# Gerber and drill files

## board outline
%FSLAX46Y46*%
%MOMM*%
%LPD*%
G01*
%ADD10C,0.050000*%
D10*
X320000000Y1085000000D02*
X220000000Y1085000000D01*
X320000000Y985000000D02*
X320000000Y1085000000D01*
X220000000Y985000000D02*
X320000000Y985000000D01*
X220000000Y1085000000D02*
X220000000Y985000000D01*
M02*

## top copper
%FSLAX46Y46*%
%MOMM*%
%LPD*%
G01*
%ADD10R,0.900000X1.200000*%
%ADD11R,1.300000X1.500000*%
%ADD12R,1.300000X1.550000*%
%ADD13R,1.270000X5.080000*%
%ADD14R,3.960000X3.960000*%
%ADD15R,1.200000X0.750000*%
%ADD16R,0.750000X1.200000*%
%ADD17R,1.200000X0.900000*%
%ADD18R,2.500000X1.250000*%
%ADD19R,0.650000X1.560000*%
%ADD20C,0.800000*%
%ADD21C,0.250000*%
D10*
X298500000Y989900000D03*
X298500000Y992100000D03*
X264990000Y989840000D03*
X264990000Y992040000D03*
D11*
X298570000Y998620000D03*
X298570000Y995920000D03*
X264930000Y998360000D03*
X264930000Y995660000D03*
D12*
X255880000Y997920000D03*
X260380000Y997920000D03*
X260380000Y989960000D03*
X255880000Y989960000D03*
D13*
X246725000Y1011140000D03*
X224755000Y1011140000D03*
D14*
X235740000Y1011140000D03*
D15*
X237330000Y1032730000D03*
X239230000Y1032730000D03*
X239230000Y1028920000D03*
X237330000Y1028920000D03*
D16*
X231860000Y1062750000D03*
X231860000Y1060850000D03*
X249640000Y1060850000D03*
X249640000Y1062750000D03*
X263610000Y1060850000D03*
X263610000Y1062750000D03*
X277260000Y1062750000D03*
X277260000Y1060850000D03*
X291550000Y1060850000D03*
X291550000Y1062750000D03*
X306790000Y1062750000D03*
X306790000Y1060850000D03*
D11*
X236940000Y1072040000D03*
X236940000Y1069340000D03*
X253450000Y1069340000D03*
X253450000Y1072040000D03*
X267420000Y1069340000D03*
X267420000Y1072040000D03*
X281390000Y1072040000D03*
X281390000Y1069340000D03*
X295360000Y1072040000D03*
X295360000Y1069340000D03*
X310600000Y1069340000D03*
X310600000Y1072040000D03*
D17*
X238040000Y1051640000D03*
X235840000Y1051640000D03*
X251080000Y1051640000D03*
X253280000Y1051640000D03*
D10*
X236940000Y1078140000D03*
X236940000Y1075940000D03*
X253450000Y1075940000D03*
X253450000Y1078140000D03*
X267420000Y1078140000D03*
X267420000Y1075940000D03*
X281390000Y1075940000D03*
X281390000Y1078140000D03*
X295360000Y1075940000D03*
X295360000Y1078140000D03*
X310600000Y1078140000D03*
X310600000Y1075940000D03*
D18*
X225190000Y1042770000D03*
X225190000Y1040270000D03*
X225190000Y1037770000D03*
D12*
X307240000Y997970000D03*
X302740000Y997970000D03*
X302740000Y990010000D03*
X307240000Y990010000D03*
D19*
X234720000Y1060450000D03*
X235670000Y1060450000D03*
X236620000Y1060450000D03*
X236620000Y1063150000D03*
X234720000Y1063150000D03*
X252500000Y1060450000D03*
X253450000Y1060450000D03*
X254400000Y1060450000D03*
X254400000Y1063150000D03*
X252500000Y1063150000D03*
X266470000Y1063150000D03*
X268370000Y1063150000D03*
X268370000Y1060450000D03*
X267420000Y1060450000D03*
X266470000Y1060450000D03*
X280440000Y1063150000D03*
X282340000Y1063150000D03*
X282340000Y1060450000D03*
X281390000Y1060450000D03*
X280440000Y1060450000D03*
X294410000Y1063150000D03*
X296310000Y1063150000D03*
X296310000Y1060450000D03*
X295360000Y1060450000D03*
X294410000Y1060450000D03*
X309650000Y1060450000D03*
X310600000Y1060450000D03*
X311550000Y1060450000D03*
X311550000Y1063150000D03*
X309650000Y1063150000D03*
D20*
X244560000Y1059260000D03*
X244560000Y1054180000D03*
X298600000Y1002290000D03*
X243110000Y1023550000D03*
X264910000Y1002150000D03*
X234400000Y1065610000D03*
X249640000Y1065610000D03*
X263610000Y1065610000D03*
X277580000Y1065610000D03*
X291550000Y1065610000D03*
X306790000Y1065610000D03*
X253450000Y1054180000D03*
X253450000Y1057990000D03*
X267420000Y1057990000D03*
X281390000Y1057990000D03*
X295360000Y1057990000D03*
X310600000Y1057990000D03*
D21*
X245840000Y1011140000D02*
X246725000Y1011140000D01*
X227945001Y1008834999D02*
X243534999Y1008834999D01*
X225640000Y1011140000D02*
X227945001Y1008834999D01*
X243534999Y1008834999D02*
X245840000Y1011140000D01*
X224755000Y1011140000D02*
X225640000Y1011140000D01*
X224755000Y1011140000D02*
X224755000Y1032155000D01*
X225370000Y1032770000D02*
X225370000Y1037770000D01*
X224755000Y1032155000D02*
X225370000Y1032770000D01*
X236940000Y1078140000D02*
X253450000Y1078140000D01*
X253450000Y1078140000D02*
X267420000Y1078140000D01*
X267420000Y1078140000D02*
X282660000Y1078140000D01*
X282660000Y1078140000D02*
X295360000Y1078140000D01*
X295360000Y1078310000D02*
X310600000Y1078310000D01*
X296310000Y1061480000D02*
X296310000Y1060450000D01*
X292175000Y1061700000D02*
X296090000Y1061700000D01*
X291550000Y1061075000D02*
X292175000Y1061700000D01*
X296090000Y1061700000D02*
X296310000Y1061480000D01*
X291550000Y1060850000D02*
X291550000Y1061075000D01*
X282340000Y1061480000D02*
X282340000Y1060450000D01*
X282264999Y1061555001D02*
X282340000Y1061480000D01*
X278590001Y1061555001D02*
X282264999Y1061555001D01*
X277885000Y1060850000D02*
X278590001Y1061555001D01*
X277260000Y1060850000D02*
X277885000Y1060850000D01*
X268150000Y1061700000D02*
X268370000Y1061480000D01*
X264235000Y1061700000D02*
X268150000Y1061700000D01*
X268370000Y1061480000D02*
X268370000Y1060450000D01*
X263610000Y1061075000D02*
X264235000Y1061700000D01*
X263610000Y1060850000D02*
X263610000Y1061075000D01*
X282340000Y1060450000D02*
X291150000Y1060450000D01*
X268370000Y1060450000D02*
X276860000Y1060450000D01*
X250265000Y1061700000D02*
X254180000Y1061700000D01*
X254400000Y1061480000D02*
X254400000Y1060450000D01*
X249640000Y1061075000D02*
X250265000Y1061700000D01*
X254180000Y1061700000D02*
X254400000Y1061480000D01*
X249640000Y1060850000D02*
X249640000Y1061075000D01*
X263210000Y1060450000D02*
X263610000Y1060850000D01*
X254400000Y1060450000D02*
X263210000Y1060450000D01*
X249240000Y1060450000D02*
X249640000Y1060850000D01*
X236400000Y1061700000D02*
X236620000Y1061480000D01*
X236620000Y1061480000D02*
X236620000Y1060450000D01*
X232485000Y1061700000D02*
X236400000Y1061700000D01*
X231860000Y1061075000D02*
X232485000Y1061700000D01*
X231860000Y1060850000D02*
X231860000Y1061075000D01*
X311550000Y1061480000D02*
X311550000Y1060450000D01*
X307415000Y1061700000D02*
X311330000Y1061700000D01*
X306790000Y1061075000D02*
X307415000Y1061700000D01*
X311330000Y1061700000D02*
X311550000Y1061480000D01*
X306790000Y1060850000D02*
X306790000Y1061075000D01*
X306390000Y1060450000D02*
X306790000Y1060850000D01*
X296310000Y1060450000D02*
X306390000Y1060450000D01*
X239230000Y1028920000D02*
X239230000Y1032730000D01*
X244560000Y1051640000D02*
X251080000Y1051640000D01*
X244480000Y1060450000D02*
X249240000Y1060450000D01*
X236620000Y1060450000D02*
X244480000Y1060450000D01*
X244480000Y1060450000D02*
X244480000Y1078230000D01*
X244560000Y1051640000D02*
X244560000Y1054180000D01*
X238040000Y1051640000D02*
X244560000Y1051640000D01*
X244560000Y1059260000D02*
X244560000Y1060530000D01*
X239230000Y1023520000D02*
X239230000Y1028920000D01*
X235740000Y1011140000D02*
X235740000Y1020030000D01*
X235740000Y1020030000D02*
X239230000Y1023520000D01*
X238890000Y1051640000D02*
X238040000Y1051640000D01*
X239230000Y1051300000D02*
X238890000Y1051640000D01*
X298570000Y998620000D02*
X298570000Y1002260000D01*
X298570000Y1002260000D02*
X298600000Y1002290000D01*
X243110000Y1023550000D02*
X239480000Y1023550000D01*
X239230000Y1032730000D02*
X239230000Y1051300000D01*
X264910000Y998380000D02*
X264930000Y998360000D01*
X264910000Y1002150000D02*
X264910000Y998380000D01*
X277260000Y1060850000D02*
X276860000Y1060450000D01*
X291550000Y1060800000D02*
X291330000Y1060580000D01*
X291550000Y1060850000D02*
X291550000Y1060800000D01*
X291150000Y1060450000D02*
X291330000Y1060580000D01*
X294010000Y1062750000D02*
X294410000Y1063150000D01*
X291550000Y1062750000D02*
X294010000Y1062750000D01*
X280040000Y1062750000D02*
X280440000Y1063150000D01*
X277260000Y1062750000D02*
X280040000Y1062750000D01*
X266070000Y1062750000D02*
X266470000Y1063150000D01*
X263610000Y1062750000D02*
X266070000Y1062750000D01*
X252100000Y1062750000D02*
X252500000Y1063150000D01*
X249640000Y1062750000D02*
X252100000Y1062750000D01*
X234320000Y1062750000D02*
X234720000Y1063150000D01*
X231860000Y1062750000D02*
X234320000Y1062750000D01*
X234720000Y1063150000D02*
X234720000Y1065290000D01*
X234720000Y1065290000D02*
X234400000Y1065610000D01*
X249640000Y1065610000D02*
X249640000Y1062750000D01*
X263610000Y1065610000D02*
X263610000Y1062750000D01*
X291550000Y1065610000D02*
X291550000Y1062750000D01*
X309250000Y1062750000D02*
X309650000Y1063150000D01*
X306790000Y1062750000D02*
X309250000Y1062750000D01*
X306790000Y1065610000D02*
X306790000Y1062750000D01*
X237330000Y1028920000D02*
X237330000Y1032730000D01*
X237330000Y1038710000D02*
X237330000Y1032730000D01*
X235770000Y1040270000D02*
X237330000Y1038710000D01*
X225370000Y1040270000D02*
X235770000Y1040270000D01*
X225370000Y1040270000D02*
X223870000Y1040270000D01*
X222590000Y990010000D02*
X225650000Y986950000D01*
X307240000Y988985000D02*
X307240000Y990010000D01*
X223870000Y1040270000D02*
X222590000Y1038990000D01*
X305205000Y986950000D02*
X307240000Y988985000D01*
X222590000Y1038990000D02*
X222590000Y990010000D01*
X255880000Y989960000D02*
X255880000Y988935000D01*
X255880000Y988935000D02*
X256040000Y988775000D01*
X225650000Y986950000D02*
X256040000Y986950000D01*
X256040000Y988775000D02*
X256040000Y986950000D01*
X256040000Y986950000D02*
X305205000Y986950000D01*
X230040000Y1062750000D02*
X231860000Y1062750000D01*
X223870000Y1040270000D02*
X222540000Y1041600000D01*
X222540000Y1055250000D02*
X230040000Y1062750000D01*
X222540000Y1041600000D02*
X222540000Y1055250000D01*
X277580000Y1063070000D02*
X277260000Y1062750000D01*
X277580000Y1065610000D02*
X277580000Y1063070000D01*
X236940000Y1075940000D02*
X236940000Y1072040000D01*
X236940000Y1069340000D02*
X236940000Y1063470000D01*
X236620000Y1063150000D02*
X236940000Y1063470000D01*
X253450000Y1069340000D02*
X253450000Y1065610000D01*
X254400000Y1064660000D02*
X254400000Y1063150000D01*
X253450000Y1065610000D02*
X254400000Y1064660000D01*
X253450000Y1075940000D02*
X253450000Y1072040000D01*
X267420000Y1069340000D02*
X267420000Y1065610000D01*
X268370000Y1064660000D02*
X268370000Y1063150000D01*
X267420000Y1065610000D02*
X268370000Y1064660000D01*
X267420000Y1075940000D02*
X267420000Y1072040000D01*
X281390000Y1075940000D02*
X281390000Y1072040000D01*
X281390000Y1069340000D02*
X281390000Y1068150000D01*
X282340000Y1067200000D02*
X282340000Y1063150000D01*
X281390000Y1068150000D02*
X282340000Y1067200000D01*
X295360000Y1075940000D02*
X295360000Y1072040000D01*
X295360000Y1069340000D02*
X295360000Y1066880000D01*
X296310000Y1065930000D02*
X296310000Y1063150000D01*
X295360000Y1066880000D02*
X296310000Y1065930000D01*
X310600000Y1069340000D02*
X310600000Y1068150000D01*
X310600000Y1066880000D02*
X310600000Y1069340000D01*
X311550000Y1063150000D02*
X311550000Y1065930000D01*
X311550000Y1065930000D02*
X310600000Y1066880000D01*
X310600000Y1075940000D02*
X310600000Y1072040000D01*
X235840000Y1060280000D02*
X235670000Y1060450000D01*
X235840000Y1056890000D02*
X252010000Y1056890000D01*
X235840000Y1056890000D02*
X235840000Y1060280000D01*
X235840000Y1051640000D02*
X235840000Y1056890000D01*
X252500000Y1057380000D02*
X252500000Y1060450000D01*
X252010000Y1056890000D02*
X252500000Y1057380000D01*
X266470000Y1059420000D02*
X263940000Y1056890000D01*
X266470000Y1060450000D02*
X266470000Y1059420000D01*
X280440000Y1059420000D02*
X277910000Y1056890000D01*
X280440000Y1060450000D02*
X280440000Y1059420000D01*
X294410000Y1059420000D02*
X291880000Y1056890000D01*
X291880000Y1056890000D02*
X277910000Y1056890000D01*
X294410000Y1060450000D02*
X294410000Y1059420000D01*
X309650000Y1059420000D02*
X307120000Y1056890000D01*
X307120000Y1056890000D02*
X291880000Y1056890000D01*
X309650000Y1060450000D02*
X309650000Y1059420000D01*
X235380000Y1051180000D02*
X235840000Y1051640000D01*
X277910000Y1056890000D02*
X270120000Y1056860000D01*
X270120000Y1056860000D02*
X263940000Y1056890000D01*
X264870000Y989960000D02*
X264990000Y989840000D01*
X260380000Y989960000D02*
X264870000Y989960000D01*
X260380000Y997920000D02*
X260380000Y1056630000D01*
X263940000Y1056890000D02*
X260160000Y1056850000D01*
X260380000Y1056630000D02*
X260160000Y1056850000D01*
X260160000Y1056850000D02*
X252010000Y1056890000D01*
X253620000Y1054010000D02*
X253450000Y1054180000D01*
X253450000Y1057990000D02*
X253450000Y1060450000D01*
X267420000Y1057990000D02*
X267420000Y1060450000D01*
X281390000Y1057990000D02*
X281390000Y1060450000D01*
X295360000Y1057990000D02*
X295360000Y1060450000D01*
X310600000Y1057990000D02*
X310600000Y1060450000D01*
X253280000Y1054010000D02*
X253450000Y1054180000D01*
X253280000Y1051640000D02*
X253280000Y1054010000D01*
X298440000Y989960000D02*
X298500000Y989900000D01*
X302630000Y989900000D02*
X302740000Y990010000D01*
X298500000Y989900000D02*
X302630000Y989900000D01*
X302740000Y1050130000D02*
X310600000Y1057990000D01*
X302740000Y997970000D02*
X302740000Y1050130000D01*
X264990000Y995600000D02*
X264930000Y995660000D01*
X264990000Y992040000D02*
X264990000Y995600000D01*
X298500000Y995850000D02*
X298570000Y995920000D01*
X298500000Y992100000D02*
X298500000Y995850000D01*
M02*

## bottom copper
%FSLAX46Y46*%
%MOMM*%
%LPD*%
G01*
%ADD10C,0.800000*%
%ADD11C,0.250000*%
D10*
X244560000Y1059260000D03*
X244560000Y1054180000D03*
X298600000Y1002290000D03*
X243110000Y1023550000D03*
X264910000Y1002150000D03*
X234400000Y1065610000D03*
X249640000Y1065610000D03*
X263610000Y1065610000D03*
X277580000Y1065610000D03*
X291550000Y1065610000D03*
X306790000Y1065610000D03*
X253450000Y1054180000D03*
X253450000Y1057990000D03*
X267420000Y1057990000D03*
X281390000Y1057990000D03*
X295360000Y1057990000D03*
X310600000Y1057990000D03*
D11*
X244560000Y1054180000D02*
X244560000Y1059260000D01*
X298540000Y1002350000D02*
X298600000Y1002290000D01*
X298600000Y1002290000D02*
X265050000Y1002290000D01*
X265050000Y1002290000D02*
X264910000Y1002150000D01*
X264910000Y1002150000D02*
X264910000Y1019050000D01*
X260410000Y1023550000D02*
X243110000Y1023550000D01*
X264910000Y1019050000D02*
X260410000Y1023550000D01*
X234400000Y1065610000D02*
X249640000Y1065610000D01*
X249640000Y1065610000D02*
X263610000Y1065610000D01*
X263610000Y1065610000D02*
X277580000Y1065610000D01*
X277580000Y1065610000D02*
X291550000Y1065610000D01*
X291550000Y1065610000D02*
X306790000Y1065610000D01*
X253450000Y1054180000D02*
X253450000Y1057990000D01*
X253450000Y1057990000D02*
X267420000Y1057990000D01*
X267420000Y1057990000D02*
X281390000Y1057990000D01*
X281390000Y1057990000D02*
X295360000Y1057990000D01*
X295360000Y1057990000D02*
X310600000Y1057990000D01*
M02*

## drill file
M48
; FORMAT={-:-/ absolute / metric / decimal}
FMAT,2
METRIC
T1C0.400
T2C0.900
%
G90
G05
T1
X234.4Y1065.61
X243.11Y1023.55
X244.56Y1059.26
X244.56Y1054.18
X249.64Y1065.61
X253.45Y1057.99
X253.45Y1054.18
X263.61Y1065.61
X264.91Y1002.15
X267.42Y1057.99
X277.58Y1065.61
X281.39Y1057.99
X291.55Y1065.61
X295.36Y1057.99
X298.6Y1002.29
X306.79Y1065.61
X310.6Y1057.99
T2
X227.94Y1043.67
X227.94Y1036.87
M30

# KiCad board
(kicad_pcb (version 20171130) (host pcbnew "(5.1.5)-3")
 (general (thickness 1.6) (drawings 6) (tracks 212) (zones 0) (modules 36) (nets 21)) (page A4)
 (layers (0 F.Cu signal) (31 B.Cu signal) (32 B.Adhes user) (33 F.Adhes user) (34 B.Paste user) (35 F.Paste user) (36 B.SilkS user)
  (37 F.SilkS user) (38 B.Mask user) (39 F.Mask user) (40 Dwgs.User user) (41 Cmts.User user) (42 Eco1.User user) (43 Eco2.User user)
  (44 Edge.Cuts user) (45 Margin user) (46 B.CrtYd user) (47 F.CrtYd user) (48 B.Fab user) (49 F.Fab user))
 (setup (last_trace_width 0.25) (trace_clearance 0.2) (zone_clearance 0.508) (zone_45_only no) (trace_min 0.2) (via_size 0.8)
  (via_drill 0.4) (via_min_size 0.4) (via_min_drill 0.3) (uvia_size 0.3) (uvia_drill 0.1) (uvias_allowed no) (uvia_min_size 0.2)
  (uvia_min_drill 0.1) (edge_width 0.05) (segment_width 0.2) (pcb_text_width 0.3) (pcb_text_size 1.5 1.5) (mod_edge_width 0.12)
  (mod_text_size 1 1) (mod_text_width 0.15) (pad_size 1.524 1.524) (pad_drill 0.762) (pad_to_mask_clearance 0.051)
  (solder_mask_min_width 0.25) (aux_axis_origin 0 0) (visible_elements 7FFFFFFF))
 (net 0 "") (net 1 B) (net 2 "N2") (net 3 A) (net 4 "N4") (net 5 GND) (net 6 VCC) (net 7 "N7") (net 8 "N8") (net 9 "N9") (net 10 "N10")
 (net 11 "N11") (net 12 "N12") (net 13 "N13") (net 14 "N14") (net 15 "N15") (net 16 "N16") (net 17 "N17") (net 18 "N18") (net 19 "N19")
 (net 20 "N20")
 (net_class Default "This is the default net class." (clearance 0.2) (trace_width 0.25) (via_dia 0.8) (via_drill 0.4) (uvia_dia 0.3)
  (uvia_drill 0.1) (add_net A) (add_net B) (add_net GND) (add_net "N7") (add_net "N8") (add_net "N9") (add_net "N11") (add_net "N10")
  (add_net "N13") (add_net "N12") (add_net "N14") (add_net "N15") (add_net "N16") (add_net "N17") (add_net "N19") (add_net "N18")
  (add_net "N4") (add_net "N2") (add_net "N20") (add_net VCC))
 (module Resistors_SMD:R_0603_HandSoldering (layer F.Cu) (at 298.5 -991 90)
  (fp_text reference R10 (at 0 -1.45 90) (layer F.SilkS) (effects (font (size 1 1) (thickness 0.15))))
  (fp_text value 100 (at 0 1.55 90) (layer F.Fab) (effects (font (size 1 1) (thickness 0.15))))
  (pad 1 smd rect (at -1.1 0 90) (size 1.2 0.9) (layers F.Cu F.Paste F.Mask) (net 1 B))
  (pad 2 smd rect (at 1.1 0 90) (size 1.2 0.9) (layers F.Cu F.Paste F.Mask) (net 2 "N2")))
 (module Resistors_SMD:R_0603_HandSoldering (layer F.Cu) (at 264.99 -990.94 90)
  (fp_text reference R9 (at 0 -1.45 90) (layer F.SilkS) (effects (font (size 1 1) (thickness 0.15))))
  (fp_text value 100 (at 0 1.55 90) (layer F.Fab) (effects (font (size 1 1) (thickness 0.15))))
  (pad 1 smd rect (at -1.1 0 90) (size 1.2 0.9) (layers F.Cu F.Paste F.Mask) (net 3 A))
  (pad 2 smd rect (at 1.1 0 90) (size 1.2 0.9) (layers F.Cu F.Paste F.Mask) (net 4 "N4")))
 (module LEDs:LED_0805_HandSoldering (layer F.Cu) (at 298.57 -997.27 270)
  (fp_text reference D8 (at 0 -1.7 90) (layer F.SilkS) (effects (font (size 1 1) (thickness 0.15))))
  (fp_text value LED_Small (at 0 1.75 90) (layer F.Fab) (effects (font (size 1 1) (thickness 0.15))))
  (pad 1 smd rect (at -1.35 0 270) (size 1.5 1.3) (layers F.Cu F.Paste F.Mask) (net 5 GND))
  (pad 2 smd rect (at 1.35 0 270) (size 1.5 1.3) (layers F.Cu F.Paste F.Mask) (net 2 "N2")))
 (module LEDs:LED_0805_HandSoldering (layer F.Cu) (at 264.93 -997.01 270)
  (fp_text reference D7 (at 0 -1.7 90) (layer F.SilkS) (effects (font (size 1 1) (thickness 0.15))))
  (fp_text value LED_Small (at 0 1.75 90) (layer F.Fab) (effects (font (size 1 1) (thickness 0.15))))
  (pad 1 smd rect (at -1.35 0 270) (size 1.5 1.3) (layers F.Cu F.Paste F.Mask) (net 5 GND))
  (pad 2 smd rect (at 1.35 0 270) (size 1.5 1.3) (layers F.Cu F.Paste F.Mask) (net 4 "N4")))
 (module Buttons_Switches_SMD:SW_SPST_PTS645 (layer F.Cu) (at 258.13 -993.94 270)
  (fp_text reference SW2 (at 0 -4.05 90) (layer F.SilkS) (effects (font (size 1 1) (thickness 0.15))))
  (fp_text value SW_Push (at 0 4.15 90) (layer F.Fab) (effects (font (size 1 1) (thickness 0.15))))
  (pad 2 smd rect (at -3.98 2.25 270) (size 1.55 1.3) (layers F.Cu F.Paste F.Mask) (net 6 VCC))
  (pad 1 smd rect (at -3.98 -2.25 270) (size 1.55 1.3) (layers F.Cu F.Paste F.Mask) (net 3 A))
  (pad 1 smd rect (at 3.98 -2.25 270) (size 1.55 1.3) (layers F.Cu F.Paste F.Mask) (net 3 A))
  (pad 2 smd rect (at 3.98 2.25 270) (size 1.55 1.3) (layers F.Cu F.Paste F.Mask) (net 6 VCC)))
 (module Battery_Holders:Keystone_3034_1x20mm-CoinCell (layer F.Cu) (at 235.74 -1011.14 180)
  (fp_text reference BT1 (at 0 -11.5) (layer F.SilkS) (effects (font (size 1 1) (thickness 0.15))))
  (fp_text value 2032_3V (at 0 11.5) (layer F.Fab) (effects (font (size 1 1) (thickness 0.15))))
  (pad 1 smd rect (at -10.985 0 180) (size 1.27 5.08) (layers F.Cu F.Paste F.Mask) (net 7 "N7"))
  (pad 1 smd rect (at 10.985 0 180) (size 1.27 5.08) (layers F.Cu F.Paste F.Mask) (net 7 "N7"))
  (pad 2 smd rect (at 0 0 180) (size 3.96 3.96) (layers F.Cu F.Paste F.Mask) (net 5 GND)))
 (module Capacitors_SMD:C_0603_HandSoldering (layer F.Cu) (at 238.28 -1032.73)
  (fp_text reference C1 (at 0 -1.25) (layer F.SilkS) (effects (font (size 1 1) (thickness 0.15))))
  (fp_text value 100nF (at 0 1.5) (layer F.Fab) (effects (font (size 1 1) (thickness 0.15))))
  (pad 1 smd rect (at -0.95 0) (size 1.2 0.75) (layers F.Cu F.Paste F.Mask) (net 6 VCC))
  (pad 2 smd rect (at 0.95 0) (size 1.2 0.75) (layers F.Cu F.Paste F.Mask) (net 5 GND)))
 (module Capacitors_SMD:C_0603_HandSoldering (layer F.Cu) (at 238.28 -1028.92)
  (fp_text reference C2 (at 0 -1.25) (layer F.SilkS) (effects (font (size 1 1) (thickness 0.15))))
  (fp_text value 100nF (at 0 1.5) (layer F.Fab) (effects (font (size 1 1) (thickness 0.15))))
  (pad 2 smd rect (at 0.95 0) (size 1.2 0.75) (layers F.Cu F.Paste F.Mask) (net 5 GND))
  (pad 1 smd rect (at -0.95 0) (size 1.2 0.75) (layers F.Cu F.Paste F.Mask) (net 6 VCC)))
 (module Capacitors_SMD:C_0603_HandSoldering (layer F.Cu) (at 231.86 -1061.8 270)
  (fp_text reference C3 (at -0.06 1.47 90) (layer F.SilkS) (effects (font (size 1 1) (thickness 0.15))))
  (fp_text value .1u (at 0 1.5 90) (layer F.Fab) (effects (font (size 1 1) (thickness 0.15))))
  (pad 1 smd rect (at -0.95 0 270) (size 1.2 0.75) (layers F.Cu F.Paste F.Mask) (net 6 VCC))
  (pad 2 smd rect (at 0.95 0 270) (size 1.2 0.75) (layers F.Cu F.Paste F.Mask) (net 5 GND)))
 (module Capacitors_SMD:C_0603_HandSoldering (layer F.Cu) (at 249.64 -1061.8 270)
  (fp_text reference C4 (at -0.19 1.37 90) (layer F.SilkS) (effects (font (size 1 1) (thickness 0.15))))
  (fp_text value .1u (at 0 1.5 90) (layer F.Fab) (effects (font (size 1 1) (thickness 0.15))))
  (pad 2 smd rect (at 0.95 0 270) (size 1.2 0.75) (layers F.Cu F.Paste F.Mask) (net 5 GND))
  (pad 1 smd rect (at -0.95 0 270) (size 1.2 0.75) (layers F.Cu F.Paste F.Mask) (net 6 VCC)))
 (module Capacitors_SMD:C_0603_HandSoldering (layer F.Cu) (at 263.61 -1061.8 270)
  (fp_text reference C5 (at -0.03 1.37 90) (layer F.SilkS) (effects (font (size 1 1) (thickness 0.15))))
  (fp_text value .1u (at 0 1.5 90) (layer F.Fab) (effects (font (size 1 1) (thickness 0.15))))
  (pad 2 smd rect (at 0.95 0 270) (size 1.2 0.75) (layers F.Cu F.Paste F.Mask) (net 5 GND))
  (pad 1 smd rect (at -0.95 0 270) (size 1.2 0.75) (layers F.Cu F.Paste F.Mask) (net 6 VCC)))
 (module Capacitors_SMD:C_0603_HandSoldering (layer F.Cu) (at 277.26 -1061.8 270)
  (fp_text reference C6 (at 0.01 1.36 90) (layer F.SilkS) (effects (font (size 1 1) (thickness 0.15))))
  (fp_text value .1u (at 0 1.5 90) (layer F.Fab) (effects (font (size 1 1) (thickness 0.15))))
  (pad 1 smd rect (at -0.95 0 270) (size 1.2 0.75) (layers F.Cu F.Paste F.Mask) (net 6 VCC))
  (pad 2 smd rect (at 0.95 0 270) (size 1.2 0.75) (layers F.Cu F.Paste F.Mask) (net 5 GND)))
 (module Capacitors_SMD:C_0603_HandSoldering (layer F.Cu) (at 291.55 -1061.8 270)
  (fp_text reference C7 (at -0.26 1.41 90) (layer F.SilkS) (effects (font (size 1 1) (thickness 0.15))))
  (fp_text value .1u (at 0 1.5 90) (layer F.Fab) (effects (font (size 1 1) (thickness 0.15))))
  (pad 2 smd rect (at 0.95 0 270) (size 1.2 0.75) (layers F.Cu F.Paste F.Mask) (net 5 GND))
  (pad 1 smd rect (at -0.95 0 270) (size 1.2 0.75) (layers F.Cu F.Paste F.Mask) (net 6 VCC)))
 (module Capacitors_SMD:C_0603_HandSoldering (layer F.Cu) (at 306.79 -1061.8 270)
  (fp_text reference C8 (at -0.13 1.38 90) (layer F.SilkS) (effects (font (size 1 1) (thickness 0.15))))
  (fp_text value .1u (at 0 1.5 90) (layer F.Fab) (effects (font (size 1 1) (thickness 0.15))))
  (pad 1 smd rect (at -0.95 0 270) (size 1.2 0.75) (layers F.Cu F.Paste F.Mask) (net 6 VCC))
  (pad 2 smd rect (at 0.95 0 270) (size 1.2 0.75) (layers F.Cu F.Paste F.Mask) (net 5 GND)))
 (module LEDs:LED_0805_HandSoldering (layer F.Cu) (at 236.94 -1070.69 270)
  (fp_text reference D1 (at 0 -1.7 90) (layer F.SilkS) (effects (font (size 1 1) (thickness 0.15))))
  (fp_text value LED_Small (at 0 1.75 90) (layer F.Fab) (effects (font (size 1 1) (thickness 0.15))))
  (pad 1 smd rect (at -1.35 0 270) (size 1.5 1.3) (layers F.Cu F.Paste F.Mask) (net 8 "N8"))
  (pad 2 smd rect (at 1.35 0 270) (size 1.5 1.3) (layers F.Cu F.Paste F.Mask) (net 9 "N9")))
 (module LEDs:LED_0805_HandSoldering (layer F.Cu) (at 253.45 -1070.69 270)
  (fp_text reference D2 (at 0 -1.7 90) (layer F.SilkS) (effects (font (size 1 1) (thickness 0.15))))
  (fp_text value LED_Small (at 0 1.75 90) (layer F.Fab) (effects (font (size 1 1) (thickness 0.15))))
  (pad 2 smd rect (at 1.35 0 270) (size 1.5 1.3) (layers F.Cu F.Paste F.Mask) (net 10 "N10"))
  (pad 1 smd rect (at -1.35 0 270) (size 1.5 1.3) (layers F.Cu F.Paste F.Mask) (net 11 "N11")))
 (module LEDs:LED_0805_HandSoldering (layer F.Cu) (at 267.42 -1070.69 270)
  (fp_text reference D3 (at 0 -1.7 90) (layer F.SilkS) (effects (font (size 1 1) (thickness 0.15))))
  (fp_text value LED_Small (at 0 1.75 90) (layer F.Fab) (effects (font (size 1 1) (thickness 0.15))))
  (pad 2 smd rect (at 1.35 0 270) (size 1.5 1.3) (layers F.Cu F.Paste F.Mask) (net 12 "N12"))
  (pad 1 smd rect (at -1.35 0 270) (size 1.5 1.3) (layers F.Cu F.Paste F.Mask) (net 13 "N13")))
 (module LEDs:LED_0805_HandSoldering (layer F.Cu) (at 281.39 -1070.69 270)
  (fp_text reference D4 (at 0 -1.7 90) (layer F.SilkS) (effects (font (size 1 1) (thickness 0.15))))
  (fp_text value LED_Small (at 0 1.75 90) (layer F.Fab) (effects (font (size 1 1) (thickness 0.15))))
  (pad 1 smd rect (at -1.35 0 270) (size 1.5 1.3) (layers F.Cu F.Paste F.Mask) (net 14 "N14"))
  (pad 2 smd rect (at 1.35 0 270) (size 1.5 1.3) (layers F.Cu F.Paste F.Mask) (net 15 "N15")))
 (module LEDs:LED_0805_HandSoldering (layer F.Cu) (at 295.36 -1070.69 270)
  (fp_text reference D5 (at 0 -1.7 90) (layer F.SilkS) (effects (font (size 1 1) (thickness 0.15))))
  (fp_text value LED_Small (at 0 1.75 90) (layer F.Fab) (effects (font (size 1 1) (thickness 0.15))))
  (pad 1 smd rect (at -1.35 0 270) (size 1.5 1.3) (layers F.Cu F.Paste F.Mask) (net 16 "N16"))
  (pad 2 smd rect (at 1.35 0 270) (size 1.5 1.3) (layers F.Cu F.Paste F.Mask) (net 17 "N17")))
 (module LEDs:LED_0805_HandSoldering (layer F.Cu) (at 310.6 -1070.69 270)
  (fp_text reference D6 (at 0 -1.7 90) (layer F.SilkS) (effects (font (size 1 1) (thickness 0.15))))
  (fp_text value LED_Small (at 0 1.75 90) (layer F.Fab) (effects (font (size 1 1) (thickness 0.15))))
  (pad 2 smd rect (at 1.35 0 270) (size 1.5 1.3) (layers F.Cu F.Paste F.Mask) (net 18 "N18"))
  (pad 1 smd rect (at -1.35 0 270) (size 1.5 1.3) (layers F.Cu F.Paste F.Mask) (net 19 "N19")))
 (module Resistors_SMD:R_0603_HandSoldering (layer F.Cu) (at 236.94 -1051.64 180)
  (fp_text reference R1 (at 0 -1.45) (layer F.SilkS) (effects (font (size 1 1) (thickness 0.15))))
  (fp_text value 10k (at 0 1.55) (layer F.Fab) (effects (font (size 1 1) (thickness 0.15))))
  (pad 1 smd rect (at -1.1 0 180) (size 1.2 0.9) (layers F.Cu F.Paste F.Mask) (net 5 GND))
  (pad 2 smd rect (at 1.1 0 180) (size 1.2 0.9) (layers F.Cu F.Paste F.Mask) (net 3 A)))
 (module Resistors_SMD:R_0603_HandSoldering (layer F.Cu) (at 252.18 -1051.64 180)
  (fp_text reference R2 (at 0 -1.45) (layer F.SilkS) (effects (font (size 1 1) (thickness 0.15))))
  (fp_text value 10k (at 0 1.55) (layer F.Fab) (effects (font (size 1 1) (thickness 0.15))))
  (pad 2 smd rect (at 1.1 0 180) (size 1.2 0.9) (layers F.Cu F.Paste F.Mask) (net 5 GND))
  (pad 1 smd rect (at -1.1 0 180) (size 1.2 0.9) (layers F.Cu F.Paste F.Mask) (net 1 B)))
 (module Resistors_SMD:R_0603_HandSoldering (layer F.Cu) (at 236.94 -1077.04 270)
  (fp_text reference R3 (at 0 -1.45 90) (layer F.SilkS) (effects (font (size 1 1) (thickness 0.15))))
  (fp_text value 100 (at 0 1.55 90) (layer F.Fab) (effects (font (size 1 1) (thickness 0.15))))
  (pad 1 smd rect (at -1.1 0 270) (size 1.2 0.9) (layers F.Cu F.Paste F.Mask) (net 5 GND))
  (pad 2 smd rect (at 1.1 0 270) (size 1.2 0.9) (layers F.Cu F.Paste F.Mask) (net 8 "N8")))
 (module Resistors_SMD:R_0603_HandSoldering (layer F.Cu) (at 253.45 -1077.04 270)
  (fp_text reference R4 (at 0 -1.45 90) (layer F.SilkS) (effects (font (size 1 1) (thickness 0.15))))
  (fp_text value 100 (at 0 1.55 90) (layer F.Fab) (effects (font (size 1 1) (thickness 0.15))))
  (pad 2 smd rect (at 1.1 0 270) (size 1.2 0.9) (layers F.Cu F.Paste F.Mask) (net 11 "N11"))
  (pad 1 smd rect (at -1.1 0 270) (size 1.2 0.9) (layers F.Cu F.Paste F.Mask) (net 5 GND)))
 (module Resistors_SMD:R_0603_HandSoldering (layer F.Cu) (at 267.42 -1077.04 270)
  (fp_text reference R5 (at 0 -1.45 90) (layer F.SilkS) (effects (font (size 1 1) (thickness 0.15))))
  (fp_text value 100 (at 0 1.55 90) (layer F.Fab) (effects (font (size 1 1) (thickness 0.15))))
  (pad 1 smd rect (at -1.1 0 270) (size 1.2 0.9) (layers F.Cu F.Paste F.Mask) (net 5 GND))
  (pad 2 smd rect (at 1.1 0 270) (size 1.2 0.9) (layers F.Cu F.Paste F.Mask) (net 13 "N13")))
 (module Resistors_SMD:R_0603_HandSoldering (layer F.Cu) (at 281.39 -1077.04 270)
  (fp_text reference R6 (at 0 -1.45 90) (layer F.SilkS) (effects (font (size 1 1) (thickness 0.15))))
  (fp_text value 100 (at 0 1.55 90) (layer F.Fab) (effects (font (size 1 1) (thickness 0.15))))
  (pad 2 smd rect (at 1.1 0 270) (size 1.2 0.9) (layers F.Cu F.Paste F.Mask) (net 14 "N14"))
  (pad 1 smd rect (at -1.1 0 270) (size 1.2 0.9) (layers F.Cu F.Paste F.Mask) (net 5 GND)))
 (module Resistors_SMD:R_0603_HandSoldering (layer F.Cu) (at 295.36 -1077.04 270)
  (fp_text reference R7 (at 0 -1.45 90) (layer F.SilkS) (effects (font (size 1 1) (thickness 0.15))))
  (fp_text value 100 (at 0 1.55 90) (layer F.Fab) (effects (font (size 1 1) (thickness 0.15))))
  (pad 2 smd rect (at 1.1 0 270) (size 1.2 0.9) (layers F.Cu F.Paste F.Mask) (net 16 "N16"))
  (pad 1 smd rect (at -1.1 0 270) (size 1.2 0.9) (layers F.Cu F.Paste F.Mask) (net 5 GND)))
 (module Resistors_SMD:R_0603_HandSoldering (layer F.Cu) (at 310.6 -1077.04 270)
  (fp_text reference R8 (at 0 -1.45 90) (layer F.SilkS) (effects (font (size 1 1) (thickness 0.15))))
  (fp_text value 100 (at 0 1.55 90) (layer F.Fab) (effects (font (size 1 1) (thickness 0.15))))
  (pad 1 smd rect (at -1.1 0 270) (size 1.2 0.9) (layers F.Cu F.Paste F.Mask) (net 5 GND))
  (pad 2 smd rect (at 1.1 0 270) (size 1.2 0.9) (layers F.Cu F.Paste F.Mask) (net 19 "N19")))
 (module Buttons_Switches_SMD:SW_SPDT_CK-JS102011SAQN (layer F.Cu) (at 227.94 -1040.27 90)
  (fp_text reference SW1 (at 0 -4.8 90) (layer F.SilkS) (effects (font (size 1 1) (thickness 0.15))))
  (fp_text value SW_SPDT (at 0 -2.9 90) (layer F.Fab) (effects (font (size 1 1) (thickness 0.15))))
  (pad "" np_thru_hole circle (at 3.4 0 90) (size 0.9 0.9) (drill 0.9) (layers *.Cu *.Mask))
  (pad "" np_thru_hole circle (at -3.4 0 90) (size 0.9 0.9) (drill 0.9) (layers *.Cu *.Mask))
  (pad 3 smd rect (at 2.5 -2.75 90) (size 1.25 2.5) (layers F.Cu F.Paste F.Mask) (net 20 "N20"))
  (pad 2 smd rect (at 0 -2.75 90) (size 1.25 2.5) (layers F.Cu F.Paste F.Mask) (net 6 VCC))
  (pad 1 smd rect (at -2.5 -2.75 90) (size 1.25 2.5) (layers F.Cu F.Paste F.Mask) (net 7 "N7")))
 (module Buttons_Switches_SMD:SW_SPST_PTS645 (layer F.Cu) (at 304.99 -993.99 90)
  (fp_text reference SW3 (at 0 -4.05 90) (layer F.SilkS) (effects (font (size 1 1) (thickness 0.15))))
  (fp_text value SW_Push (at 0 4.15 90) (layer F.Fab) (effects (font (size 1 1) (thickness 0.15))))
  (pad 2 smd rect (at 3.98 2.25 90) (size 1.55 1.3) (layers F.Cu F.Paste F.Mask) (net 6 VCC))
  (pad 1 smd rect (at 3.98 -2.25 90) (size 1.55 1.3) (layers F.Cu F.Paste F.Mask) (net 1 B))
  (pad 1 smd rect (at -3.98 -2.25 90) (size 1.55 1.3) (layers F.Cu F.Paste F.Mask) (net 1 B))
  (pad 2 smd rect (at -3.98 2.25 90) (size 1.55 1.3) (layers F.Cu F.Paste F.Mask) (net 6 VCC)))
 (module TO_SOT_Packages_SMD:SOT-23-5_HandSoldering (layer F.Cu) (at 235.67 -1061.8 90)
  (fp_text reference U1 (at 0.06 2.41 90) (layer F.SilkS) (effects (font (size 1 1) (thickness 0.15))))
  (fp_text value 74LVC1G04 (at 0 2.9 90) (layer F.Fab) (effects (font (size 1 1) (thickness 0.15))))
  (pad 1 smd rect (at -1.35 -0.95 90) (size 1.56 0.65) (layers F.Cu F.Paste F.Mask))
  (pad 2 smd rect (at -1.35 0 90) (size 1.56 0.65) (layers F.Cu F.Paste F.Mask) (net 3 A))
  (pad 3 smd rect (at -1.35 0.95 90) (size 1.56 0.65) (layers F.Cu F.Paste F.Mask) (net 5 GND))
  (pad 4 smd rect (at 1.35 0.95 90) (size 1.56 0.65) (layers F.Cu F.Paste F.Mask) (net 9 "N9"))
  (pad 5 smd rect (at 1.35 -0.95 90) (size 1.56 0.65) (layers F.Cu F.Paste F.Mask) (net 6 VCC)))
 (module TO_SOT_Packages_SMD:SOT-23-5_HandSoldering (layer F.Cu) (at 253.45 -1061.8 90)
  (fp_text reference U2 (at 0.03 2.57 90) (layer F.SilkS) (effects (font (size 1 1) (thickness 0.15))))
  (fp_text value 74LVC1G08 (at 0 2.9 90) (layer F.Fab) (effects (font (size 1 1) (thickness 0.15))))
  (pad 1 smd rect (at -1.35 -0.95 90) (size 1.56 0.65) (layers F.Cu F.Paste F.Mask) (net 3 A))
  (pad 2 smd rect (at -1.35 0 90) (size 1.56 0.65) (layers F.Cu F.Paste F.Mask) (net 1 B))
  (pad 3 smd rect (at -1.35 0.95 90) (size 1.56 0.65) (layers F.Cu F.Paste F.Mask) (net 5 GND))
  (pad 4 smd rect (at 1.35 0.95 90) (size 1.56 0.65) (layers F.Cu F.Paste F.Mask) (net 10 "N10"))
  (pad 5 smd rect (at 1.35 -0.95 90) (size 1.56 0.65) (layers F.Cu F.Paste F.Mask) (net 6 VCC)))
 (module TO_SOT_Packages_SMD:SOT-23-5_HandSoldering (layer F.Cu) (at 267.42 -1061.8 90)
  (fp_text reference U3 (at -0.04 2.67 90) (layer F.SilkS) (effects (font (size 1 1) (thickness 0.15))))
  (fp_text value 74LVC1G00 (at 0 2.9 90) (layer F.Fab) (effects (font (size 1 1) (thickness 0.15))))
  (pad 5 smd rect (at 1.35 -0.95 90) (size 1.56 0.65) (layers F.Cu F.Paste F.Mask) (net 6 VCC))
  (pad 4 smd rect (at 1.35 0.95 90) (size 1.56 0.65) (layers F.Cu F.Paste F.Mask) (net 12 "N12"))
  (pad 3 smd rect (at -1.35 0.95 90) (size 1.56 0.65) (layers F.Cu F.Paste F.Mask) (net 5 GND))
  (pad 2 smd rect (at -1.35 0 90) (size 1.56 0.65) (layers F.Cu F.Paste F.Mask) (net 1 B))
  (pad 1 smd rect (at -1.35 -0.95 90) (size 1.56 0.65) (layers F.Cu F.Paste F.Mask) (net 3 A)))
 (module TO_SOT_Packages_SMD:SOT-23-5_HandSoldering (layer F.Cu) (at 281.39 -1061.8 90)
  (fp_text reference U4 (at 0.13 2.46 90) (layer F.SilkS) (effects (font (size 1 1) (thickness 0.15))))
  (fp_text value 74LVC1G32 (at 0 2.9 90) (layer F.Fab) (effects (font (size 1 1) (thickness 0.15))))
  (pad 5 smd rect (at 1.35 -0.95 90) (size 1.56 0.65) (layers F.Cu F.Paste F.Mask) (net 6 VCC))
  (pad 4 smd rect (at 1.35 0.95 90) (size 1.56 0.65) (layers F.Cu F.Paste F.Mask) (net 15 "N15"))
  (pad 3 smd rect (at -1.35 0.95 90) (size 1.56 0.65) (layers F.Cu F.Paste F.Mask) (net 5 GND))
  (pad 2 smd rect (at -1.35 0 90) (size 1.56 0.65) (layers F.Cu F.Paste F.Mask) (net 1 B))
  (pad 1 smd rect (at -1.35 -0.95 90) (size 1.56 0.65) (layers F.Cu F.Paste F.Mask) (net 3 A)))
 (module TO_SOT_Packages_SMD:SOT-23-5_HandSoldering (layer F.Cu) (at 295.36 -1061.8 90)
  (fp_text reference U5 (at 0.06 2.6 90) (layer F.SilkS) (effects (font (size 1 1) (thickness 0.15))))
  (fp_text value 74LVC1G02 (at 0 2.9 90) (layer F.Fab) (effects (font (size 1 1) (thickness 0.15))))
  (pad 5 smd rect (at 1.35 -0.95 90) (size 1.56 0.65) (layers F.Cu F.Paste F.Mask) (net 6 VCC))
  (pad 4 smd rect (at 1.35 0.95 90) (size 1.56 0.65) (layers F.Cu F.Paste F.Mask) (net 17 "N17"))
  (pad 3 smd rect (at -1.35 0.95 90) (size 1.56 0.65) (layers F.Cu F.Paste F.Mask) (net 5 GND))
  (pad 2 smd rect (at -1.35 0 90) (size 1.56 0.65) (layers F.Cu F.Paste F.Mask) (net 1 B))
  (pad 1 smd rect (at -1.35 -0.95 90) (size 1.56 0.65) (layers F.Cu F.Paste F.Mask) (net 3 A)))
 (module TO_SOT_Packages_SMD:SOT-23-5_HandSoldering (layer F.Cu) (at 310.6 -1061.8 90)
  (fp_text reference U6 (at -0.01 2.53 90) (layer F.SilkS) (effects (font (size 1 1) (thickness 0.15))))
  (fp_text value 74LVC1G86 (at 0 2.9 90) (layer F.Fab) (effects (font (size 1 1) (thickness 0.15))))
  (pad 1 smd rect (at -1.35 -0.95 90) (size 1.56 0.65) (layers F.Cu F.Paste F.Mask) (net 3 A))
  (pad 2 smd rect (at -1.35 0 90) (size 1.56 0.65) (layers F.Cu F.Paste F.Mask) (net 1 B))
  (pad 3 smd rect (at -1.35 0.95 90) (size 1.56 0.65) (layers F.Cu F.Paste F.Mask) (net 5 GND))
  (pad 4 smd rect (at 1.35 0.95 90) (size 1.56 0.65) (layers F.Cu F.Paste F.Mask) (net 18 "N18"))
  (pad 5 smd rect (at 1.35 -0.95 90) (size 1.56 0.65) (layers F.Cu F.Paste F.Mask) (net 6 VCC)))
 (gr_line (start 320 -1085) (end 220 -1085) (layer Edge.Cuts) (width 0.05))
 (gr_line (start 320 -985) (end 320 -1085) (layer Edge.Cuts) (width 0.05))
 (gr_line (start 220 -985) (end 320 -985) (layer Edge.Cuts) (width 0.05))
 (gr_line (start 220 -1085) (end 220 -985) (layer Edge.Cuts) (width 0.05))
 (segment (start 245.84 -1011.14) (end 246.725 -1011.14) (width 0.25) (layer F.Cu) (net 7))
 (segment (start 227.945001 -1008.834999) (end 243.534999 -1008.834999) (width 0.25) (layer F.Cu) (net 7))
 (segment (start 225.64 -1011.14) (end 227.945001 -1008.834999) (width 0.25) (layer F.Cu) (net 7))
 (segment (start 243.534999 -1008.834999) (end 245.84 -1011.14) (width 0.25) (layer F.Cu) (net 7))
 (segment (start 224.755 -1011.14) (end 225.64 -1011.14) (width 0.25) (layer F.Cu) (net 7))
 (segment (start 224.755 -1011.14) (end 224.755 -1032.155) (width 0.25) (layer F.Cu) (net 7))
 (segment (start 225.37 -1032.77) (end 225.37 -1037.77) (width 0.25) (layer F.Cu) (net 7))
 (segment (start 224.755 -1032.155) (end 225.37 -1032.77) (width 0.25) (layer F.Cu) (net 7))
 (segment (start 236.94 -1078.14) (end 253.45 -1078.14) (width 0.25) (layer F.Cu) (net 5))
 (segment (start 253.45 -1078.14) (end 267.42 -1078.14) (width 0.25) (layer F.Cu) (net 5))
 (segment (start 267.42 -1078.14) (end 282.66 -1078.14) (width 0.25) (layer F.Cu) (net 5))
 (segment (start 282.66 -1078.14) (end 295.36 -1078.14) (width 0.25) (layer F.Cu) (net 5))
 (segment (start 295.36 -1078.31) (end 310.6 -1078.31) (width 0.25) (layer F.Cu) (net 5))
 (segment (start 296.31 -1061.48) (end 296.31 -1060.45) (width 0.25) (layer F.Cu) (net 5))
 (segment (start 292.175 -1061.7) (end 296.09 -1061.7) (width 0.25) (layer F.Cu) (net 5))
 (segment (start 291.55 -1061.075) (end 292.175 -1061.7) (width 0.25) (layer F.Cu) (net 5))
 (segment (start 296.09 -1061.7) (end 296.31 -1061.48) (width 0.25) (layer F.Cu) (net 5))
 (segment (start 291.55 -1060.85) (end 291.55 -1061.075) (width 0.25) (layer F.Cu) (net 5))
 (segment (start 282.34 -1061.48) (end 282.34 -1060.45) (width 0.25) (layer F.Cu) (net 5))
 (segment (start 282.264999 -1061.555001) (end 282.34 -1061.48) (width 0.25) (layer F.Cu) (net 5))
 (segment (start 278.590001 -1061.555001) (end 282.264999 -1061.555001) (width 0.25) (layer F.Cu) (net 5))
 (segment (start 277.885 -1060.85) (end 278.590001 -1061.555001) (width 0.25) (layer F.Cu) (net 5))
 (segment (start 277.26 -1060.85) (end 277.885 -1060.85) (width 0.25) (layer F.Cu) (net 5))
 (segment (start 268.15 -1061.7) (end 268.37 -1061.48) (width 0.25) (layer F.Cu) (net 5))
 (segment (start 264.235 -1061.7) (end 268.15 -1061.7) (width 0.25) (layer F.Cu) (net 5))
 (segment (start 268.37 -1061.48) (end 268.37 -1060.45) (width 0.25) (layer F.Cu) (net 5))
 (segment (start 263.61 -1061.075) (end 264.235 -1061.7) (width 0.25) (layer F.Cu) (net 5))
 (segment (start 263.61 -1060.85) (end 263.61 -1061.075) (width 0.25) (layer F.Cu) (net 5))
 (segment (start 282.34 -1060.45) (end 291.15 -1060.45) (width 0.25) (layer F.Cu) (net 5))
 (segment (start 268.37 -1060.45) (end 276.86 -1060.45) (width 0.25) (layer F.Cu) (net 5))
 (segment (start 250.265 -1061.7) (end 254.18 -1061.7) (width 0.25) (layer F.Cu) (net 5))
 (segment (start 254.4 -1061.48) (end 254.4 -1060.45) (width 0.25) (layer F.Cu) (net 5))
 (segment (start 249.64 -1061.075) (end 250.265 -1061.7) (width 0.25) (layer F.Cu) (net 5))
 (segment (start 254.18 -1061.7) (end 254.4 -1061.48) (width 0.25) (layer F.Cu) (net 5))
 (segment (start 249.64 -1060.85) (end 249.64 -1061.075) (width 0.25) (layer F.Cu) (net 5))
 (segment (start 263.21 -1060.45) (end 263.61 -1060.85) (width 0.25) (layer F.Cu) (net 5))
 (segment (start 254.4 -1060.45) (end 263.21 -1060.45) (width 0.25) (layer F.Cu) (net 5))
 (segment (start 249.24 -1060.45) (end 249.64 -1060.85) (width 0.25) (layer F.Cu) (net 5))
 (segment (start 236.4 -1061.7) (end 236.62 -1061.48) (width 0.25) (layer F.Cu) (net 5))
 (segment (start 236.62 -1061.48) (end 236.62 -1060.45) (width 0.25) (layer F.Cu) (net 5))
 (segment (start 232.485 -1061.7) (end 236.4 -1061.7) (width 0.25) (layer F.Cu) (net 5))
 (segment (start 231.86 -1061.075) (end 232.485 -1061.7) (width 0.25) (layer F.Cu) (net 5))
 (segment (start 231.86 -1060.85) (end 231.86 -1061.075) (width 0.25) (layer F.Cu) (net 5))
 (segment (start 311.55 -1061.48) (end 311.55 -1060.45) (width 0.25) (layer F.Cu) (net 5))
 (segment (start 307.415 -1061.7) (end 311.33 -1061.7) (width 0.25) (layer F.Cu) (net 5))
 (segment (start 306.79 -1061.075) (end 307.415 -1061.7) (width 0.25) (layer F.Cu) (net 5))
 (segment (start 311.33 -1061.7) (end 311.55 -1061.48) (width 0.25) (layer F.Cu) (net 5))
 (segment (start 306.79 -1060.85) (end 306.79 -1061.075) (width 0.25) (layer F.Cu) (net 5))
 (segment (start 306.39 -1060.45) (end 306.79 -1060.85) (width 0.25) (layer F.Cu) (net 5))
 (segment (start 296.31 -1060.45) (end 306.39 -1060.45) (width 0.25) (layer F.Cu) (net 5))
 (segment (start 239.23 -1028.92) (end 239.23 -1032.73) (width 0.25) (layer F.Cu) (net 5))
 (segment (start 244.56 -1051.64) (end 251.08 -1051.64) (width 0.25) (layer F.Cu) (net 5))
 (segment (start 244.48 -1060.45) (end 249.24 -1060.45) (width 0.25) (layer F.Cu) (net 5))
 (segment (start 236.62 -1060.45) (end 244.48 -1060.45) (width 0.25) (layer F.Cu) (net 5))
 (segment (start 244.48 -1060.45) (end 244.48 -1078.23) (width 0.25) (layer F.Cu) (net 5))
 (via (at 244.56 -1059.26) (size 0.8) (drill 0.4) (layers F.Cu B.Cu) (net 5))
 (via (at 244.56 -1054.18) (size 0.8) (drill 0.4) (layers F.Cu B.Cu) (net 5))
 (segment (start 244.56 -1051.64) (end 244.56 -1054.18) (width 0.25) (layer F.Cu) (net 5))
 (segment (start 238.04 -1051.64) (end 244.56 -1051.64) (width 0.25) (layer F.Cu) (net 5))
 (segment (start 244.56 -1054.18) (end 244.56 -1059.26) (width 0.25) (layer B.Cu) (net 5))
 (segment (start 244.56 -1059.26) (end 244.56 -1060.53) (width 0.25) (layer F.Cu) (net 5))
 (segment (start 239.23 -1023.52) (end 239.23 -1028.92) (width 0.25) (layer F.Cu) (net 5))
 (segment (start 235.74 -1011.14) (end 235.74 -1020.03) (width 0.25) (layer F.Cu) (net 5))
 (segment (start 235.74 -1020.03) (end 239.23 -1023.52) (width 0.25) (layer F.Cu) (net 5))
 (segment (start 238.89 -1051.64) (end 238.04 -1051.64) (width 0.25) (layer F.Cu) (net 5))
 (segment (start 239.23 -1051.3) (end 238.89 -1051.64) (width 0.25) (layer F.Cu) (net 5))
 (via (at 298.6 -1002.29) (size 0.8) (drill 0.4) (layers F.Cu B.Cu) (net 5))
 (segment (start 298.57 -998.62) (end 298.57 -1002.26) (width 0.25) (layer F.Cu) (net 5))
 (segment (start 298.57 -1002.26) (end 298.6 -1002.29) (width 0.25) (layer F.Cu) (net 5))
 (via (at 243.11 -1023.55) (size 0.8) (drill 0.4) (layers F.Cu B.Cu) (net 5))
 (segment (start 243.11 -1023.55) (end 239.48 -1023.55) (width 0.25) (layer F.Cu) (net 5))
 (segment (start 298.54 -1002.35) (end 298.6 -1002.29) (width 0.25) (layer B.Cu) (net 5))
 (segment (start 239.23 -1032.73) (end 239.23 -1051.3) (width 0.25) (layer F.Cu) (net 5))
 (via (at 264.91 -1002.15) (size 0.8) (drill 0.4) (layers F.Cu B.Cu) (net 5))
 (segment (start 298.6 -1002.29) (end 265.05 -1002.29) (width 0.25) (layer B.Cu) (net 5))
 (segment (start 265.05 -1002.29) (end 264.91 -1002.15) (width 0.25) (layer B.Cu) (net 5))
 (segment (start 264.91 -998.38) (end 264.93 -998.36) (width 0.25) (layer F.Cu) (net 5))
 (segment (start 264.91 -1002.15) (end 264.91 -998.38) (width 0.25) (layer F.Cu) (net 5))
 (segment (start 264.91 -1002.15) (end 264.91 -1019.05) (width 0.25) (layer B.Cu) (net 5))
 (segment (start 260.41 -1023.55) (end 243.11 -1023.55) (width 0.25) (layer B.Cu) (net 5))
 (segment (start 264.91 -1019.05) (end 260.41 -1023.55) (width 0.25) (layer B.Cu) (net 5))
 (segment (start 277.26 -1060.85) (end 276.86 -1060.45) (width 0.25) (layer F.Cu) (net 5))
 (segment (start 291.55 -1060.8) (end 291.33 -1060.58) (width 0.25) (layer F.Cu) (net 5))
 (segment (start 291.55 -1060.85) (end 291.55 -1060.8) (width 0.25) (layer F.Cu) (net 5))
 (segment (start 291.15 -1060.45) (end 291.33 -1060.58) (width 0.25) (layer F.Cu) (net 5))
 (segment (start 294.01 -1062.75) (end 294.41 -1063.15) (width 0.25) (layer F.Cu) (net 6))
 (segment (start 291.55 -1062.75) (end 294.01 -1062.75) (width 0.25) (layer F.Cu) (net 6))
 (segment (start 280.04 -1062.75) (end 280.44 -1063.15) (width 0.25) (layer F.Cu) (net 6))
 (segment (start 277.26 -1062.75) (end 280.04 -1062.75) (width 0.25) (layer F.Cu) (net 6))
 (segment (start 266.07 -1062.75) (end 266.47 -1063.15) (width 0.25) (layer F.Cu) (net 6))
 (segment (start 263.61 -1062.75) (end 266.07 -1062.75) (width 0.25) (layer F.Cu) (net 6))
 (segment (start 252.1 -1062.75) (end 252.5 -1063.15) (width 0.25) (layer F.Cu) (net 6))
 (segment (start 249.64 -1062.75) (end 252.1 -1062.75) (width 0.25) (layer F.Cu) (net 6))
 (segment (start 234.32 -1062.75) (end 234.72 -1063.15) (width 0.25) (layer F.Cu) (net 6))
 (segment (start 231.86 -1062.75) (end 234.32 -1062.75) (width 0.25) (layer F.Cu) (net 6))
 (via (at 234.4 -1065.61) (size 0.8) (drill 0.4) (layers F.Cu B.Cu) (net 6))
 (segment (start 234.72 -1063.15) (end 234.72 -1065.29) (width 0.25) (layer F.Cu) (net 6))
 (segment (start 234.72 -1065.29) (end 234.4 -1065.61) (width 0.25) (layer F.Cu) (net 6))
 (via (at 249.64 -1065.61) (size 0.8) (drill 0.4) (layers F.Cu B.Cu) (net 6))
 (segment (start 234.4 -1065.61) (end 249.64 -1065.61) (width 0.25) (layer B.Cu) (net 6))
 (segment (start 249.64 -1065.61) (end 249.64 -1062.75) (width 0.25) (layer F.Cu) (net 6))
 (via (at 263.61 -1065.61) (size 0.8) (drill 0.4) (layers F.Cu B.Cu) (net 6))
 (segment (start 249.64 -1065.61) (end 263.61 -1065.61) (width 0.25) (layer B.Cu) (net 6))
 (segment (start 263.61 -1065.61) (end 263.61 -1062.75) (width 0.25) (layer F.Cu) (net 6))
 (via (at 277.58 -1065.61) (size 0.8) (drill 0.4) (layers F.Cu B.Cu) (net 6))
 (segment (start 263.61 -1065.61) (end 277.58 -1065.61) (width 0.25) (layer B.Cu) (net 6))
 (via (at 291.55 -1065.61) (size 0.8) (drill 0.4) (layers F.Cu B.Cu) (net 6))
 (segment (start 277.58 -1065.61) (end 291.55 -1065.61) (width 0.25) (layer B.Cu) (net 6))
 (segment (start 291.55 -1065.61) (end 291.55 -1062.75) (width 0.25) (layer F.Cu) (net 6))
 (segment (start 309.25 -1062.75) (end 309.65 -1063.15) (width 0.25) (layer F.Cu) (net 6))
 (segment (start 306.79 -1062.75) (end 309.25 -1062.75) (width 0.25) (layer F.Cu) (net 6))
 (via (at 306.79 -1065.61) (size 0.8) (drill 0.4) (layers F.Cu B.Cu) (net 6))
 (segment (start 291.55 -1065.61) (end 306.79 -1065.61) (width 0.25) (layer B.Cu) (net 6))
 (segment (start 306.79 -1065.61) (end 306.79 -1062.75) (width 0.25) (layer F.Cu) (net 6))
 (segment (start 237.33 -1028.92) (end 237.33 -1032.73) (width 0.25) (layer F.Cu) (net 6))
 (segment (start 237.33 -1038.71) (end 237.33 -1032.73) (width 0.25) (layer F.Cu) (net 6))
 (segment (start 235.77 -1040.27) (end 237.33 -1038.71) (width 0.25) (layer F.Cu) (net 6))
 (segment (start 225.37 -1040.27) (end 235.77 -1040.27) (width 0.25) (layer F.Cu) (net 6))
 (segment (start 225.37 -1040.27) (end 223.87 -1040.27) (width 0.25) (layer F.Cu) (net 6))
 (segment (start 222.59 -990.01) (end 225.65 -986.95) (width 0.25) (layer F.Cu) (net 6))
 (segment (start 307.24 -988.985) (end 307.24 -990.01) (width 0.25) (layer F.Cu) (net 6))
 (segment (start 223.87 -1040.27) (end 222.59 -1038.99) (width 0.25) (layer F.Cu) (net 6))
 (segment (start 305.205 -986.95) (end 307.24 -988.985) (width 0.25) (layer F.Cu) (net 6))
 (segment (start 222.59 -1038.99) (end 222.59 -990.01) (width 0.25) (layer F.Cu) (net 6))
 (segment (start 255.88 -989.96) (end 255.88 -988.935) (width 0.25) (layer F.Cu) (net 6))
 (segment (start 255.88 -988.935) (end 256.04 -988.775) (width 0.25) (layer F.Cu) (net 6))
 (segment (start 225.65 -986.95) (end 256.04 -986.95) (width 0.25) (layer F.Cu) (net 6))
 (segment (start 256.04 -988.775) (end 256.04 -986.95) (width 0.25) (layer F.Cu) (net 6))
 (segment (start 256.04 -986.95) (end 305.205 -986.95) (width 0.25) (layer F.Cu) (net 6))
 (segment (start 230.04 -1062.75) (end 231.86 -1062.75) (width 0.25) (layer F.Cu) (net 6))
 (segment (start 223.87 -1040.27) (end 222.54 -1041.6) (width 0.25) (layer F.Cu) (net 6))
 (segment (start 222.54 -1055.25) (end 230.04 -1062.75) (width 0.25) (layer F.Cu) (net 6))
 (segment (start 222.54 -1041.6) (end 222.54 -1055.25) (width 0.25) (layer F.Cu) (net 6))
 (segment (start 277.58 -1063.07) (end 277.26 -1062.75) (width 0.25) (layer F.Cu) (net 6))
 (segment (start 277.58 -1065.61) (end 277.58 -1063.07) (width 0.25) (layer F.Cu) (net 6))
 (segment (start 236.94 -1075.94) (end 236.94 -1072.04) (width 0.25) (layer F.Cu) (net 8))
 (segment (start 236.94 -1069.34) (end 236.94 -1063.47) (width 0.25) (layer F.Cu) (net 9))
 (segment (start 236.62 -1063.15) (end 236.94 -1063.47) (width 0.25) (layer F.Cu) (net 9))
 (segment (start 253.45 -1069.34) (end 253.45 -1065.61) (width 0.25) (layer F.Cu) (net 10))
 (segment (start 254.4 -1064.66) (end 254.4 -1063.15) (width 0.25) (layer F.Cu) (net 10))
 (segment (start 253.45 -1065.61) (end 254.4 -1064.66) (width 0.25) (layer F.Cu) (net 10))
 (segment (start 253.45 -1075.94) (end 253.45 -1072.04) (width 0.25) (layer F.Cu) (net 11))
 (segment (start 267.42 -1069.34) (end 267.42 -1065.61) (width 0.25) (layer F.Cu) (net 12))
 (segment (start 268.37 -1064.66) (end 268.37 -1063.15) (width 0.25) (layer F.Cu) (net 12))
 (segment (start 267.42 -1065.61) (end 268.37 -1064.66) (width 0.25) (layer F.Cu) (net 12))
 (segment (start 267.42 -1075.94) (end 267.42 -1072.04) (width 0.25) (layer F.Cu) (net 13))
 (segment (start 281.39 -1075.94) (end 281.39 -1072.04) (width 0.25) (layer F.Cu) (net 14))
 (segment (start 281.39 -1069.34) (end 281.39 -1068.15) (width 0.25) (layer F.Cu) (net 15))
 (segment (start 282.34 -1067.2) (end 282.34 -1063.15) (width 0.25) (layer F.Cu) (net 15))
 (segment (start 281.39 -1068.15) (end 282.34 -1067.2) (width 0.25) (layer F.Cu) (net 15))
 (segment (start 295.36 -1075.94) (end 295.36 -1072.04) (width 0.25) (layer F.Cu) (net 16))
 (segment (start 295.36 -1069.34) (end 295.36 -1066.88) (width 0.25) (layer F.Cu) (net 17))
 (segment (start 296.31 -1065.93) (end 296.31 -1063.15) (width 0.25) (layer F.Cu) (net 17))
 (segment (start 295.36 -1066.88) (end 296.31 -1065.93) (width 0.25) (layer F.Cu) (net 17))
 (segment (start 310.6 -1069.34) (end 310.6 -1068.15) (width 0.25) (layer F.Cu) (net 18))
 (segment (start 310.6 -1066.88) (end 310.6 -1069.34) (width 0.25) (layer F.Cu) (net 18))
 (segment (start 311.55 -1063.15) (end 311.55 -1065.93) (width 0.25) (layer F.Cu) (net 18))
 (segment (start 311.55 -1065.93) (end 310.6 -1066.88) (width 0.25) (layer F.Cu) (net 18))
 (segment (start 310.6 -1075.94) (end 310.6 -1072.04) (width 0.25) (layer F.Cu) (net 19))
 (segment (start 235.84 -1060.28) (end 235.67 -1060.45) (width 0.25) (layer F.Cu) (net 3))
 (segment (start 235.84 -1056.89) (end 252.01 -1056.89) (width 0.25) (layer F.Cu) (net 3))
 (segment (start 235.84 -1056.89) (end 235.84 -1060.28) (width 0.25) (layer F.Cu) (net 3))
 (segment (start 235.84 -1051.64) (end 235.84 -1056.89) (width 0.25) (layer F.Cu) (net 3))
 (segment (start 252.5 -1057.38) (end 252.5 -1060.45) (width 0.25) (layer F.Cu) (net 3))
 (segment (start 252.01 -1056.89) (end 252.5 -1057.38) (width 0.25) (layer F.Cu) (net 3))
 (segment (start 266.47 -1059.42) (end 263.94 -1056.89) (width 0.25) (layer F.Cu) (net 3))
 (segment (start 266.47 -1060.45) (end 266.47 -1059.42) (width 0.25) (layer F.Cu) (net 3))
 (segment (start 280.44 -1059.42) (end 277.91 -1056.89) (width 0.25) (layer F.Cu) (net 3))
 (segment (start 280.44 -1060.45) (end 280.44 -1059.42) (width 0.25) (layer F.Cu) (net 3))
 (segment (start 294.41 -1059.42) (end 291.88 -1056.89) (width 0.25) (layer F.Cu) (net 3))
 (segment (start 291.88 -1056.89) (end 277.91 -1056.89) (width 0.25) (layer F.Cu) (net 3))
 (segment (start 294.41 -1060.45) (end 294.41 -1059.42) (width 0.25) (layer F.Cu) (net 3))
 (segment (start 309.65 -1059.42) (end 307.12 -1056.89) (width 0.25) (layer F.Cu) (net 3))
 (segment (start 307.12 -1056.89) (end 291.88 -1056.89) (width 0.25) (layer F.Cu) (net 3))
 (segment (start 309.65 -1060.45) (end 309.65 -1059.42) (width 0.25) (layer F.Cu) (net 3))
 (segment (start 235.38 -1051.18) (end 235.84 -1051.64) (width 0.25) (layer F.Cu) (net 3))
 (segment (start 277.91 -1056.89) (end 270.12 -1056.86) (width 0.25) (layer F.Cu) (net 3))
 (segment (start 270.12 -1056.86) (end 263.94 -1056.89) (width 0.25) (layer F.Cu) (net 3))
 (segment (start 264.87 -989.96) (end 264.99 -989.84) (width 0.25) (layer F.Cu) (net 3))
 (segment (start 260.38 -989.96) (end 264.87 -989.96) (width 0.25) (layer F.Cu) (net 3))
 (segment (start 260.38 -997.92) (end 260.38 -1056.63) (width 0.25) (layer F.Cu) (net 3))
 (segment (start 263.94 -1056.89) (end 260.16 -1056.85) (width 0.25) (layer F.Cu) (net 3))
 (segment (start 260.38 -1056.63) (end 260.16 -1056.85) (width 0.25) (layer F.Cu) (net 3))
 (segment (start 260.16 -1056.85) (end 252.01 -1056.89) (width 0.25) (layer F.Cu) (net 3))
 (via (at 253.45 -1054.18) (size 0.8) (drill 0.4) (layers F.Cu B.Cu) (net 1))
 (segment (start 253.62 -1054.01) (end 253.45 -1054.18) (width 0.25) (layer F.Cu) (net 1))
 (via (at 253.45 -1057.99) (size 0.8) (drill 0.4) (layers F.Cu B.Cu) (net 1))
 (segment (start 253.45 -1054.18) (end 253.45 -1057.99) (width 0.25) (layer B.Cu) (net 1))
 (segment (start 253.45 -1057.99) (end 253.45 -1060.45) (width 0.25) (layer F.Cu) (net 1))
 (via (at 267.42 -1057.99) (size 0.8) (drill 0.4) (layers F.Cu B.Cu) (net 1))
 (segment (start 253.45 -1057.99) (end 267.42 -1057.99) (width 0.25) (layer B.Cu) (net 1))
 (segment (start 267.42 -1057.99) (end 267.42 -1060.45) (width 0.25) (layer F.Cu) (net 1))
 (via (at 281.39 -1057.99) (size 0.8) (drill 0.4) (layers F.Cu B.Cu) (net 1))
 (segment (start 267.42 -1057.99) (end 281.39 -1057.99) (width 0.25) (layer B.Cu) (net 1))
 (segment (start 281.39 -1057.99) (end 281.39 -1060.45) (width 0.25) (layer F.Cu) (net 1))
 (via (at 295.36 -1057.99) (size 0.8) (drill 0.4) (layers F.Cu B.Cu) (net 1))
 (segment (start 281.39 -1057.99) (end 295.36 -1057.99) (width 0.25) (layer B.Cu) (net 1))
 (segment (start 295.36 -1057.99) (end 295.36 -1060.45) (width 0.25) (layer F.Cu) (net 1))
 (via (at 310.6 -1057.99) (size 0.8) (drill 0.4) (layers F.Cu B.Cu) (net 1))
 (segment (start 295.36 -1057.99) (end 310.6 -1057.99) (width 0.25) (layer B.Cu) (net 1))
 (segment (start 310.6 -1057.99) (end 310.6 -1060.45) (width 0.25) (layer F.Cu) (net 1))
 (segment (start 253.28 -1054.01) (end 253.45 -1054.18) (width 0.25) (layer F.Cu) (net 1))
 (segment (start 253.28 -1051.64) (end 253.28 -1054.01) (width 0.25) (layer F.Cu) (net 1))
 (segment (start 298.44 -989.96) (end 298.5 -989.9) (width 0.25) (layer F.Cu) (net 1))
 (segment (start 302.63 -989.9) (end 302.74 -990.01) (width 0.25) (layer F.Cu) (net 1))
 (segment (start 298.5 -989.9) (end 302.63 -989.9) (width 0.25) (layer F.Cu) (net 1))
 (segment (start 302.74 -1050.13) (end 310.6 -1057.99) (width 0.25) (layer F.Cu) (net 1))
 (segment (start 302.74 -997.97) (end 302.74 -1050.13) (width 0.25) (layer F.Cu) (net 1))
 (segment (start 264.99 -995.6) (end 264.93 -995.66) (width 0.25) (layer F.Cu) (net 4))
 (segment (start 264.99 -992.04) (end 264.99 -995.6) (width 0.25) (layer F.Cu) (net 4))
 (segment (start 298.5 -995.85) (end 298.57 -995.92) (width 0.25) (layer F.Cu) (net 2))
 (segment (start 298.5 -992.1) (end 298.5 -995.85) (width 0.25) (layer F.Cu) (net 2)))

